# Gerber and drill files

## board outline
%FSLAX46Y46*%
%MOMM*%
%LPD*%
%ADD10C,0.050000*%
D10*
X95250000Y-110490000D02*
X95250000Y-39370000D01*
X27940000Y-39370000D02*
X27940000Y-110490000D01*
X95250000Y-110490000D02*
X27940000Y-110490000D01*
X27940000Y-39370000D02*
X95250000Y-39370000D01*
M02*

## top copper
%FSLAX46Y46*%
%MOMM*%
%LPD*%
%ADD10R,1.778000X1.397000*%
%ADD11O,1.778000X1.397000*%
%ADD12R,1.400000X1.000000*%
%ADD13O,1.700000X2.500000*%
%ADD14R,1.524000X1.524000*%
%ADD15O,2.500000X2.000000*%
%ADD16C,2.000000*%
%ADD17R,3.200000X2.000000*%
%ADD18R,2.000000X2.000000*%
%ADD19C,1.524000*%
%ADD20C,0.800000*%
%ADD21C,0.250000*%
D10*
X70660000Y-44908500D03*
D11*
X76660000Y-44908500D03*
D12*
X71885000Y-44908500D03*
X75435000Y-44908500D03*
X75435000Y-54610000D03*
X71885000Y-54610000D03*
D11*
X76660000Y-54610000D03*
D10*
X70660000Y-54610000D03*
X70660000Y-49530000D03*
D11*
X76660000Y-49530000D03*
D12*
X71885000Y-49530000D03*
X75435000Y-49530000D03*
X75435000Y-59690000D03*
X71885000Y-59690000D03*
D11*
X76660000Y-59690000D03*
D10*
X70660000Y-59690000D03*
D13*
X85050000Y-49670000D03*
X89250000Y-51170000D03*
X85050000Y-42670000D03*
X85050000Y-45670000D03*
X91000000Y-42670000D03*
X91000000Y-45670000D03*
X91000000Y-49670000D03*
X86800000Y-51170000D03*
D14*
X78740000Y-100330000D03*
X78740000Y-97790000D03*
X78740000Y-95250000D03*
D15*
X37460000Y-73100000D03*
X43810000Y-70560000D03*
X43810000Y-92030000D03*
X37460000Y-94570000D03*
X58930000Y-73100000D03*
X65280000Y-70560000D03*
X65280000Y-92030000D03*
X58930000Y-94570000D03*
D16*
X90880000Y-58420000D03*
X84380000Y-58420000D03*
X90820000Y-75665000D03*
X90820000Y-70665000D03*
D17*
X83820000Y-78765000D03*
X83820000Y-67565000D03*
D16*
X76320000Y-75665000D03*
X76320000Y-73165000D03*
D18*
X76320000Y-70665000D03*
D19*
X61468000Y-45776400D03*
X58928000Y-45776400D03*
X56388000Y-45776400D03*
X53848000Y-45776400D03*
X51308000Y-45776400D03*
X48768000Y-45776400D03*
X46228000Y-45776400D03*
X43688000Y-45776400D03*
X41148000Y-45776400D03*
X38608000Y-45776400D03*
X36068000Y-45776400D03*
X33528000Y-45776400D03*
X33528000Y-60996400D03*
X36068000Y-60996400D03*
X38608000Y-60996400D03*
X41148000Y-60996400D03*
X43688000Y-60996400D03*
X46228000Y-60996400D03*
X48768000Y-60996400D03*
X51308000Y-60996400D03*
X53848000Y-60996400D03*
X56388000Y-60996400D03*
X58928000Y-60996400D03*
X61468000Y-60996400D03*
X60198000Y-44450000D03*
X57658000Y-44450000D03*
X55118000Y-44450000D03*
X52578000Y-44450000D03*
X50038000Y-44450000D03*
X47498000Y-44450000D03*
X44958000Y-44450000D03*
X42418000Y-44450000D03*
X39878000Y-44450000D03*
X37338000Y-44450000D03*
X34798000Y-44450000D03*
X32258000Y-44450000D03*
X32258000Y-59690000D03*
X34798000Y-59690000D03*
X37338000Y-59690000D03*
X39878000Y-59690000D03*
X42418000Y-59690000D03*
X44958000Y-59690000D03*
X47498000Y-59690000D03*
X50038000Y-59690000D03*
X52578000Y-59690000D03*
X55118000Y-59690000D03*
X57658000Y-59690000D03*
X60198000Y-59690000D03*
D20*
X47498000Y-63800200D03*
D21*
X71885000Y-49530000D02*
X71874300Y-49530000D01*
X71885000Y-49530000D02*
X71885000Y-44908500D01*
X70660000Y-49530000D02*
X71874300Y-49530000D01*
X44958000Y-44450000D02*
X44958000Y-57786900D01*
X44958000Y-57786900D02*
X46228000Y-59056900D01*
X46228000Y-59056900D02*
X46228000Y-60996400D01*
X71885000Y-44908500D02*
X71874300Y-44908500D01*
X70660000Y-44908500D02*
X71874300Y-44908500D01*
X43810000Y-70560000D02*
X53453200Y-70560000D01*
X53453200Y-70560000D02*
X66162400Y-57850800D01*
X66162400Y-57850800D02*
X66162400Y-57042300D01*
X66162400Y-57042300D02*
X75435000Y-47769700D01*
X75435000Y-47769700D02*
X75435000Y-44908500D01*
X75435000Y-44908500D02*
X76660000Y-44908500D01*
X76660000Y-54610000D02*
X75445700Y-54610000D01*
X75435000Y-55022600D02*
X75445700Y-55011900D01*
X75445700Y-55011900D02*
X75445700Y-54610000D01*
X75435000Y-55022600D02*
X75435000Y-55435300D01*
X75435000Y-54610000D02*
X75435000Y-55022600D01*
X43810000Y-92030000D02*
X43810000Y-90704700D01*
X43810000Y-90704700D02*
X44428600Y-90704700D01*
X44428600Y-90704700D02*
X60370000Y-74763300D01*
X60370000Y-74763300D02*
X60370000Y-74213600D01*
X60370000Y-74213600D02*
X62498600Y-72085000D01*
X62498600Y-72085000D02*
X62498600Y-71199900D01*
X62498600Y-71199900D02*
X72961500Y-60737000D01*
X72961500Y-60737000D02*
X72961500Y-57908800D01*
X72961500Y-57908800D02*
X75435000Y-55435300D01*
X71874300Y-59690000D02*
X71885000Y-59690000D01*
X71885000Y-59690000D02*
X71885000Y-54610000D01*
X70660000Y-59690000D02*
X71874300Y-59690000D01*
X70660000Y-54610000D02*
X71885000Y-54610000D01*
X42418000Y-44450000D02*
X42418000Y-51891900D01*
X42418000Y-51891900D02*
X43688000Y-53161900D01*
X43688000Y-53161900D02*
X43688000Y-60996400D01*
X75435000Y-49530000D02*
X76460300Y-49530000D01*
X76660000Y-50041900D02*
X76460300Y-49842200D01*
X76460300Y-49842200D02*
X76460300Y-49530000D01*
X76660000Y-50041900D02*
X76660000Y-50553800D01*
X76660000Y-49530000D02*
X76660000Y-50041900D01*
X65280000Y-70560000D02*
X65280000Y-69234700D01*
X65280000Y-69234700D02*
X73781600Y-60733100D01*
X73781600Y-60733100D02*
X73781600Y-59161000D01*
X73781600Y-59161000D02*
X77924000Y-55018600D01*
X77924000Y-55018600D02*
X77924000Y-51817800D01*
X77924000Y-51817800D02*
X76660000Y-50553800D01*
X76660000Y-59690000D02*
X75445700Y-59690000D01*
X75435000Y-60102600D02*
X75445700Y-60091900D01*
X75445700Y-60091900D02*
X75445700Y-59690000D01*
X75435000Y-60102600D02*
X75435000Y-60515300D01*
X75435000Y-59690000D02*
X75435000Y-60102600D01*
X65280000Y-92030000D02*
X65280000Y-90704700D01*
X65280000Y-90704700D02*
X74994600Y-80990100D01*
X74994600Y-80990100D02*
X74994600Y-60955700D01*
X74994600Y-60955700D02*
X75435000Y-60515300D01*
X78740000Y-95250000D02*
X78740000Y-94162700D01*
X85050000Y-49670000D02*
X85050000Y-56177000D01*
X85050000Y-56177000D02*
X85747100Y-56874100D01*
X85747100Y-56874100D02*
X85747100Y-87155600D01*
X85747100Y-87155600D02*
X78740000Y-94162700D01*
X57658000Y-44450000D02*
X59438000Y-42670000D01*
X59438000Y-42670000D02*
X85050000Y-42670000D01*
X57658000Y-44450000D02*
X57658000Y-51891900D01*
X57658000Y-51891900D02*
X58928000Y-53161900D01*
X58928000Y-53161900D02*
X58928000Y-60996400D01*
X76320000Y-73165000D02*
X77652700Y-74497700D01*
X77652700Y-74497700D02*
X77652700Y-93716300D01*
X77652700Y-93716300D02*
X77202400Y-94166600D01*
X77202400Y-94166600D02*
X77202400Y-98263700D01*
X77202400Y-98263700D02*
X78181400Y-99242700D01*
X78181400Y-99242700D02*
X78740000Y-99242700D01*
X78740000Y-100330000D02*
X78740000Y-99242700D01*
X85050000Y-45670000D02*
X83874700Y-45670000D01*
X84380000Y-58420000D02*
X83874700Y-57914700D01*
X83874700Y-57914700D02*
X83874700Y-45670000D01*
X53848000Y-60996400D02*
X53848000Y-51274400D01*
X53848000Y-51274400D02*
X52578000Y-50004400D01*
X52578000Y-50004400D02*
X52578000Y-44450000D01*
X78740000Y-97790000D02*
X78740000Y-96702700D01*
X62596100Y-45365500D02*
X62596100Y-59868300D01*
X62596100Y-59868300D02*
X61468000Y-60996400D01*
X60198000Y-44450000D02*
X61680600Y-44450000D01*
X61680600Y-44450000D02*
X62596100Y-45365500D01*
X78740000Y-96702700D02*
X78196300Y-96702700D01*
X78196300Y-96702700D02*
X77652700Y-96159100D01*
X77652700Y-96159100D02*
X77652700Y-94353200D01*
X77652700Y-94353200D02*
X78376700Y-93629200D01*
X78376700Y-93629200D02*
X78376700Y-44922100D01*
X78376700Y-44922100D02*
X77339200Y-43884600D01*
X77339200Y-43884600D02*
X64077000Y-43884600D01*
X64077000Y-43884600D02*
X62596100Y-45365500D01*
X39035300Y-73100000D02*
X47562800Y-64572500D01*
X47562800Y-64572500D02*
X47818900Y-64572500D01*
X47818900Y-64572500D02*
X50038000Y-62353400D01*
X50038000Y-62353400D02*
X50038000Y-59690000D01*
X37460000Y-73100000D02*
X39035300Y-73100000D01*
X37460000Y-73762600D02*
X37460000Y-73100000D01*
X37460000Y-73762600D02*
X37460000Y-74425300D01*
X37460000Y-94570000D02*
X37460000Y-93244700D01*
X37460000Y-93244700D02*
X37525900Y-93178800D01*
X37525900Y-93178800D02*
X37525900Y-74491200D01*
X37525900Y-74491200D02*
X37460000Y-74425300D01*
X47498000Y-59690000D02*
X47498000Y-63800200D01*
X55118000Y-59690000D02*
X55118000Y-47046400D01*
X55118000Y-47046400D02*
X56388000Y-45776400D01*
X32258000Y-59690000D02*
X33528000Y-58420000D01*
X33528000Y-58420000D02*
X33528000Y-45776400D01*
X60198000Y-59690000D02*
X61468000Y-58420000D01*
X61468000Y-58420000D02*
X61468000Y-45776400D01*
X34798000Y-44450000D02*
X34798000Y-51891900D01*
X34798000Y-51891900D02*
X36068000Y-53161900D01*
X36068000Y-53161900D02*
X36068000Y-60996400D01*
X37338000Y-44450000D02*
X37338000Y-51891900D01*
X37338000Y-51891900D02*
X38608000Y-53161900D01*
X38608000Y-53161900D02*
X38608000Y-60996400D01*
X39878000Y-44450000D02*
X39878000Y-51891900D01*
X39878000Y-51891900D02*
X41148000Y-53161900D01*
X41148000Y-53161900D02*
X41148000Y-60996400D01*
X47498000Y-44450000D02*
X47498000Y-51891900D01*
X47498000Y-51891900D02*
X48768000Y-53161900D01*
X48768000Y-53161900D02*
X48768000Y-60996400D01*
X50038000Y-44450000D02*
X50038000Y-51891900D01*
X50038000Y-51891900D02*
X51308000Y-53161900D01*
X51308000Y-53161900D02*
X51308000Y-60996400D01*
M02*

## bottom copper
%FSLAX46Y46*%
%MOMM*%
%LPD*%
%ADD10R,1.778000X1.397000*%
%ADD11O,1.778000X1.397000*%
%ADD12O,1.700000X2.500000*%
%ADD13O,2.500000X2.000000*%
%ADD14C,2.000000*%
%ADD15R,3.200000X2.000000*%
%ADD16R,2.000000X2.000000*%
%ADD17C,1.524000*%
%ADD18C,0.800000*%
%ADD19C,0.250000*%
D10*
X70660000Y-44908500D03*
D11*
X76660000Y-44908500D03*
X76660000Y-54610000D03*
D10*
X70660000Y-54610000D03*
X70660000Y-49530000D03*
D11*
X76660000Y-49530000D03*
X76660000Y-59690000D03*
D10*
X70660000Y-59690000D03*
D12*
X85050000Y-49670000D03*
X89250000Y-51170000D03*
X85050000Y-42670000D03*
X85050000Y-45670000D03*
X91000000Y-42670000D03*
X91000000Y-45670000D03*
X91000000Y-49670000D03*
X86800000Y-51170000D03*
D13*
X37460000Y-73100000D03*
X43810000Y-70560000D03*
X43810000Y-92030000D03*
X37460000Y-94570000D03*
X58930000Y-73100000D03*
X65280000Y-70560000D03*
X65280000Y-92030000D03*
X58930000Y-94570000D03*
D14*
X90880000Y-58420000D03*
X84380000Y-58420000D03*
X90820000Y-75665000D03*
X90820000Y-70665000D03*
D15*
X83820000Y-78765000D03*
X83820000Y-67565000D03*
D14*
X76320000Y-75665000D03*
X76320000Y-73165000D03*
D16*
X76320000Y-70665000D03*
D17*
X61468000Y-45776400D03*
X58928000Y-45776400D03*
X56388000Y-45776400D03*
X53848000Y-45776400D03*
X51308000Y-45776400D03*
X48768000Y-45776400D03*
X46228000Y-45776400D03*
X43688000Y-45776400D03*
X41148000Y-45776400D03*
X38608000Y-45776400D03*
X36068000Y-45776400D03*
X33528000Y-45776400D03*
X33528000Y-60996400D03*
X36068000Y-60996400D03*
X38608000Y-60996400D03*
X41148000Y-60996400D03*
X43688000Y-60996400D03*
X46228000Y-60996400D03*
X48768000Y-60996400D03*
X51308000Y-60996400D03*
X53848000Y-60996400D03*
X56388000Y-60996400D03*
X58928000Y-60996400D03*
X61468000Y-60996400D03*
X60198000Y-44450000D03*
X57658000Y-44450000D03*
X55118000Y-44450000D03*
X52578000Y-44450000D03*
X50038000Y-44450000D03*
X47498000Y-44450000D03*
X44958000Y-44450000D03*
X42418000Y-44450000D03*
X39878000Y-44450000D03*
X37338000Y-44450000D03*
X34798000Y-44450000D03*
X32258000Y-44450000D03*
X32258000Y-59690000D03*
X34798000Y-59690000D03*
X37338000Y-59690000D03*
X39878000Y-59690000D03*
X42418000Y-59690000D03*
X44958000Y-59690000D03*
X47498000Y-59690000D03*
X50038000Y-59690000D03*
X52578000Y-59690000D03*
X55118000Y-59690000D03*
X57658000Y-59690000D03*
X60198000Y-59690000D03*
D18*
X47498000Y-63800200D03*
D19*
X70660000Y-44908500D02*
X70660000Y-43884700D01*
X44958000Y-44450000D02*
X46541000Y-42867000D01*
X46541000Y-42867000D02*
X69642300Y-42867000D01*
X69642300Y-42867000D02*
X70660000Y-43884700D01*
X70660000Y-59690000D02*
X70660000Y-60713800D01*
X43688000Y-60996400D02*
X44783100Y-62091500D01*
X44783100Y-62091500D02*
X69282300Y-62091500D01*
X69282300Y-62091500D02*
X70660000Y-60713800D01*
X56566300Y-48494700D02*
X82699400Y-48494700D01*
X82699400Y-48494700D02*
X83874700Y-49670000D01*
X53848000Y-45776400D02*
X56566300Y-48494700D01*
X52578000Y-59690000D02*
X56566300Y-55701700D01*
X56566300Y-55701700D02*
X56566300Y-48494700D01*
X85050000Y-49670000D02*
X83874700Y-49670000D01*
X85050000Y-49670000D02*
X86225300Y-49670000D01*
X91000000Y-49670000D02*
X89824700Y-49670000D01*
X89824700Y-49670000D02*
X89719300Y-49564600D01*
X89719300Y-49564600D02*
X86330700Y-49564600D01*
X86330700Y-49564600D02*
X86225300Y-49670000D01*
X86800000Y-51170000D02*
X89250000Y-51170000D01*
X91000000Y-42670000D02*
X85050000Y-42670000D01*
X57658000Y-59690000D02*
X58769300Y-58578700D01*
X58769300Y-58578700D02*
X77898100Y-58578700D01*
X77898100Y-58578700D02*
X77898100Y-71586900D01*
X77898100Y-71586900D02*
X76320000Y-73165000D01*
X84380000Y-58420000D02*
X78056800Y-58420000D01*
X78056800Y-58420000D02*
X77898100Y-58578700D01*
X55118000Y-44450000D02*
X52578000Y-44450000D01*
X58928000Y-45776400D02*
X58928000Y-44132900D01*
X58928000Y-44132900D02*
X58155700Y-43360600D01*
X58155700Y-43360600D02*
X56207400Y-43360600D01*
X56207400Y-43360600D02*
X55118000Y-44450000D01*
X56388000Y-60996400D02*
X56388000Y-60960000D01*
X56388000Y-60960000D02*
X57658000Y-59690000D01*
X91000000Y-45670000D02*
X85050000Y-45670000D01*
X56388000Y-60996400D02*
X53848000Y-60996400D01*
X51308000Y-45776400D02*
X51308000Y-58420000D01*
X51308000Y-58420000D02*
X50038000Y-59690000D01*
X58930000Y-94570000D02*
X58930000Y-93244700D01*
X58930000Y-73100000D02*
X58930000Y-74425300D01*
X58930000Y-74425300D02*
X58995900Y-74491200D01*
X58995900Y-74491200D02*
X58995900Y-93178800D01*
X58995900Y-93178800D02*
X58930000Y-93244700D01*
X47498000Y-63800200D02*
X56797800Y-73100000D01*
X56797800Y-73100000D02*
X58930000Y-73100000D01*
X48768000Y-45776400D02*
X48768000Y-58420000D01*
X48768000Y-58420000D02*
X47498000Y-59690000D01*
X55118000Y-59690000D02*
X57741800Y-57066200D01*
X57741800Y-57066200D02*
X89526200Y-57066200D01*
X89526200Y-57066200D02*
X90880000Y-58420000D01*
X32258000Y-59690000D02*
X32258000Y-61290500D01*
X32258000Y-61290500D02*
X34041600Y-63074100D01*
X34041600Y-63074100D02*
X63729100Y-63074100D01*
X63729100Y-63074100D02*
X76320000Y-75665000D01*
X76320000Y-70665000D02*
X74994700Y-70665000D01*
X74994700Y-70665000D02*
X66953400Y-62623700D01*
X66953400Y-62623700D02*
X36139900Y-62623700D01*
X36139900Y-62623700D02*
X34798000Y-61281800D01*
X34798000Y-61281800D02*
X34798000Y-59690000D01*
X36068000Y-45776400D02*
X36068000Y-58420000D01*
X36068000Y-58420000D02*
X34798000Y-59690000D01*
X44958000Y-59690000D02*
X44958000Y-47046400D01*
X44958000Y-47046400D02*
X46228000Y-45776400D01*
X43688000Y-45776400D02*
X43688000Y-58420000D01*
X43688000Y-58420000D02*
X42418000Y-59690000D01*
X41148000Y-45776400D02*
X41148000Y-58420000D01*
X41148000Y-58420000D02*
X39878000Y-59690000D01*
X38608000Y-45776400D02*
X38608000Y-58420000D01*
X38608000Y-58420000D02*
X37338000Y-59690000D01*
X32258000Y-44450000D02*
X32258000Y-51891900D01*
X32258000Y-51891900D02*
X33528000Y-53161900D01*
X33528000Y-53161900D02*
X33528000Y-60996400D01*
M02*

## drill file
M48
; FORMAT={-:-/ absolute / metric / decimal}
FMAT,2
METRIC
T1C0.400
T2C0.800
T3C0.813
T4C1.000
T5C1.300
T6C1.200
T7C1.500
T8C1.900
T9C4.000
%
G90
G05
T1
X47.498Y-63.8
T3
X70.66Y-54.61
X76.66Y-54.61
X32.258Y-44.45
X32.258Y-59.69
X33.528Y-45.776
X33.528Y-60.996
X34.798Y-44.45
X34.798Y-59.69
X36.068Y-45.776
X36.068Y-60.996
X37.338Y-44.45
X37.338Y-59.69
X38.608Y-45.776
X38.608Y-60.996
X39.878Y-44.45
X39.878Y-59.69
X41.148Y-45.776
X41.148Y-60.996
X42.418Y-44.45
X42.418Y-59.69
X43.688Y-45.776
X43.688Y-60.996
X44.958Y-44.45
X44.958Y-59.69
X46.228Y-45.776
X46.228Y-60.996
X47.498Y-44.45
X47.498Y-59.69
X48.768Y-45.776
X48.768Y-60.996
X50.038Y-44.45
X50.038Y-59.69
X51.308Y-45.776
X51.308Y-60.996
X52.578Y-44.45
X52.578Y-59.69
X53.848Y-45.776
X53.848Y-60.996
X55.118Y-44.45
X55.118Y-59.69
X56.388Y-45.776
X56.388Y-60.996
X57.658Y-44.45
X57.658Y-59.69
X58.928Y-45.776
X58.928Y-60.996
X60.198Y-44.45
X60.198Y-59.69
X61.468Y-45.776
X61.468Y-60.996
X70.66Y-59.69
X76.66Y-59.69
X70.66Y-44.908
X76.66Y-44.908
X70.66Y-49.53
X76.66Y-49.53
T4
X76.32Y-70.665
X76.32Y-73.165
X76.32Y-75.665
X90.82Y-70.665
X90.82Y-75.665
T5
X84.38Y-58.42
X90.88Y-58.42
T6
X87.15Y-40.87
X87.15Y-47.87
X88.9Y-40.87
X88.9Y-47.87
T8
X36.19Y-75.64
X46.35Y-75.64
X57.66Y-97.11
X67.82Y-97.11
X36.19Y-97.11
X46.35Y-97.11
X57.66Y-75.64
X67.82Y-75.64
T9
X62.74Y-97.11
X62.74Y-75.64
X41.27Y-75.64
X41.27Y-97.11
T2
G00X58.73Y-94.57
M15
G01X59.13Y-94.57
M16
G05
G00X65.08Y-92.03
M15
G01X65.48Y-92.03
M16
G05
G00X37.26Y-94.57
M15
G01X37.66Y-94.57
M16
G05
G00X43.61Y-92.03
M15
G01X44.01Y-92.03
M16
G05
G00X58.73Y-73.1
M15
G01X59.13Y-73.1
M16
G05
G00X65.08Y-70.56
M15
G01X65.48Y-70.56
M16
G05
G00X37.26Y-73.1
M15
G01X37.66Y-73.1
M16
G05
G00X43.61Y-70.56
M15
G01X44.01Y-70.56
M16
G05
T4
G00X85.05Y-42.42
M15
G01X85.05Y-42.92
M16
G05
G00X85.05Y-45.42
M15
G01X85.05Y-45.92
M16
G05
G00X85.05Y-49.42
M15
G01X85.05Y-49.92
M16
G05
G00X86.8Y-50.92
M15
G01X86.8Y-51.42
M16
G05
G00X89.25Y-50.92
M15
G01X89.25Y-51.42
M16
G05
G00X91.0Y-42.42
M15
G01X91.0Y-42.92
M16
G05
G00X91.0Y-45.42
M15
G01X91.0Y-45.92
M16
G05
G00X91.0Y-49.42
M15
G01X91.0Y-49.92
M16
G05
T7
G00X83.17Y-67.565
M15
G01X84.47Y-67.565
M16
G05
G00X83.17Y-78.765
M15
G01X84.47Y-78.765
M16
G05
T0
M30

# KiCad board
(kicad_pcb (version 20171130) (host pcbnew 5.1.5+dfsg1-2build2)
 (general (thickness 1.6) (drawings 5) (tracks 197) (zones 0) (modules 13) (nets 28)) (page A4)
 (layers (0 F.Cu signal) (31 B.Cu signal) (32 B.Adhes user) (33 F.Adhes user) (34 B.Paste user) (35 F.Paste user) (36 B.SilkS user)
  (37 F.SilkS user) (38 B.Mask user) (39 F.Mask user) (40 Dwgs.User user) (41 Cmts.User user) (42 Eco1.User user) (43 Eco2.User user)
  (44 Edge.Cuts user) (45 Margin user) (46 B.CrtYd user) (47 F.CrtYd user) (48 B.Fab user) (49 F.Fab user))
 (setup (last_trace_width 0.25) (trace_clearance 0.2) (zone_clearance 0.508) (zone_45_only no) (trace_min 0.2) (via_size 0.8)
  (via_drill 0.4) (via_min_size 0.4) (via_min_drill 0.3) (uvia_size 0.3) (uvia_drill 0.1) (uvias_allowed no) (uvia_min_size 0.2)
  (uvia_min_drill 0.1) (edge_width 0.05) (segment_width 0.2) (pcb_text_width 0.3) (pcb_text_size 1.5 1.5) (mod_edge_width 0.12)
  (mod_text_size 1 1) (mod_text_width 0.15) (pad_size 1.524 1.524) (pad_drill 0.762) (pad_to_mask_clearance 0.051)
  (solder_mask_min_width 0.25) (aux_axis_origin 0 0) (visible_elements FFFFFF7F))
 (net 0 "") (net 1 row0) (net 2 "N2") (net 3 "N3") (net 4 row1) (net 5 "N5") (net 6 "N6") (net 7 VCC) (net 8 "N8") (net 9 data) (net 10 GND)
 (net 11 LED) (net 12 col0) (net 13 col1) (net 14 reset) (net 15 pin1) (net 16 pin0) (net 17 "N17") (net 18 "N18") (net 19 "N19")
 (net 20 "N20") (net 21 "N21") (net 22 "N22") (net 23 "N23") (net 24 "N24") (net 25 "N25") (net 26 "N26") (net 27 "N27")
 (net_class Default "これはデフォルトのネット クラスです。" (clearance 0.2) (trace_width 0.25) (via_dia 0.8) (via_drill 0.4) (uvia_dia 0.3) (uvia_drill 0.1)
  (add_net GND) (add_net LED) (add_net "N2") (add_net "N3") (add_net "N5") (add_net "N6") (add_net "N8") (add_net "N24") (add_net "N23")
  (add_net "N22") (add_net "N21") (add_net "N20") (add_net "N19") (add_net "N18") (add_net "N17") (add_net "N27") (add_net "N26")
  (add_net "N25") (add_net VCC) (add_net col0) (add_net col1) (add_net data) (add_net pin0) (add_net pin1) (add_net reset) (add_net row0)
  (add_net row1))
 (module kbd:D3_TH (layer F.Cu) (at 73.66 44.9085) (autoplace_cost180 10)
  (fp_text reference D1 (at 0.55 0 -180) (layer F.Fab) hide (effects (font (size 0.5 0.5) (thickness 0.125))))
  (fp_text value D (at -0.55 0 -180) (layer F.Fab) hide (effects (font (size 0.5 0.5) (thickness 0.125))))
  (pad 1 thru_hole rect (at -3 0) (size 1.778 1.397) (drill 0.8128) (layers *.Cu B.Mask) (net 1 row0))
  (pad 2 thru_hole oval (at 3 0) (size 1.778 1.397) (drill 0.8128) (layers *.Cu B.Mask) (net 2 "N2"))
  (pad 1 smd rect (at -1.775 0 180) (size 1.4 1) (layers F.Cu F.Paste F.Mask) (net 1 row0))
  (pad 2 smd rect (at 1.775 0 180) (size 1.4 1) (layers F.Cu F.Paste F.Mask) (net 2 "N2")))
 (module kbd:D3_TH (layer F.Cu) (at 73.66 54.61) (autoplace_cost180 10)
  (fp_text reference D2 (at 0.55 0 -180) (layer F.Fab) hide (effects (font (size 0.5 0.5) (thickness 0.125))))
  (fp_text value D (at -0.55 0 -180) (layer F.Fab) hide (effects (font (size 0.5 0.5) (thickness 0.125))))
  (pad 2 smd rect (at 1.775 0 180) (size 1.4 1) (layers F.Cu F.Paste F.Mask) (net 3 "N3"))
  (pad 1 smd rect (at -1.775 0 180) (size 1.4 1) (layers F.Cu F.Paste F.Mask) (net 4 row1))
  (pad 2 thru_hole oval (at 3 0) (size 1.778 1.397) (drill 0.8128) (layers *.Cu B.Mask) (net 3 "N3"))
  (pad 1 thru_hole rect (at -3 0) (size 1.778 1.397) (drill 0.8128) (layers *.Cu B.Mask) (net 4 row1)))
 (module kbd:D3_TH (layer F.Cu) (at 73.66 49.53) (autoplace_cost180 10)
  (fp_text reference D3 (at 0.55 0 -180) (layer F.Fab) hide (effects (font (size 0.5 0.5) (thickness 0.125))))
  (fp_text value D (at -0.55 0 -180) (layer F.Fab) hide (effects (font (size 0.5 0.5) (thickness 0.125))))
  (pad 1 thru_hole rect (at -3 0) (size 1.778 1.397) (drill 0.8128) (layers *.Cu B.Mask) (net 1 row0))
  (pad 2 thru_hole oval (at 3 0) (size 1.778 1.397) (drill 0.8128) (layers *.Cu B.Mask) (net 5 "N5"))
  (pad 1 smd rect (at -1.775 0 180) (size 1.4 1) (layers F.Cu F.Paste F.Mask) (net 1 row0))
  (pad 2 smd rect (at 1.775 0 180) (size 1.4 1) (layers F.Cu F.Paste F.Mask) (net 5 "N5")))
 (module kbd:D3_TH (layer F.Cu) (at 73.66 59.69) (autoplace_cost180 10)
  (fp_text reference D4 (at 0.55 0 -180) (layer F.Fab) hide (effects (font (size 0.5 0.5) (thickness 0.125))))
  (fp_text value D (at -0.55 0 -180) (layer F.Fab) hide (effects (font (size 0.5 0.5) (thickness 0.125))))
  (pad 2 smd rect (at 1.775 0 180) (size 1.4 1) (layers F.Cu F.Paste F.Mask) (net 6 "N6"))
  (pad 1 smd rect (at -1.775 0 180) (size 1.4 1) (layers F.Cu F.Paste F.Mask) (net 4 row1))
  (pad 2 thru_hole oval (at 3 0) (size 1.778 1.397) (drill 0.8128) (layers *.Cu B.Mask) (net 6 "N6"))
  (pad 1 thru_hole rect (at -3 0) (size 1.778 1.397) (drill 0.8128) (layers *.Cu B.Mask) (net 4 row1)))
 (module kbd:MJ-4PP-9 (layer F.Cu) (at 88.9 39.37)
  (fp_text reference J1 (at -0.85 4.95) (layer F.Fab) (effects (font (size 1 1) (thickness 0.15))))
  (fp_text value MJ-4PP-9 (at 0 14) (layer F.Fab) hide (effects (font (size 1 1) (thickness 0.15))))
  (pad "" np_thru_hole circle (at -1.75 8.5) (size 1.2 1.2) (drill 1.2) (layers *.Cu *.Mask F.SilkS))
  (pad "" np_thru_hole circle (at -1.75 1.5) (size 1.2 1.2) (drill 1.2) (layers *.Cu *.Mask F.SilkS))
  (pad D thru_hole oval (at -3.85 10.3) (size 1.7 2.5) (drill oval 1 1.5) (layers *.Cu *.Mask F.SilkS) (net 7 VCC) (clearance 0.15))
  (pad A thru_hole oval (at 0.35 11.8) (size 1.7 2.5) (drill oval 1 1.5) (layers *.Cu *.Mask F.SilkS) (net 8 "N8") (clearance 0.15))
  (pad B thru_hole oval (at -3.85 3.3) (size 1.7 2.5) (drill oval 1 1.5) (layers *.Cu *.Mask F.SilkS) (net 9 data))
  (pad C thru_hole oval (at -3.85 6.3) (size 1.7 2.5) (drill oval 1 1.5) (layers *.Cu *.Mask F.SilkS) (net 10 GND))
  (pad "" np_thru_hole circle (at 0 1.5) (size 1.2 1.2) (drill 1.2) (layers *.Cu *.Mask F.SilkS))
  (pad "" np_thru_hole circle (at 0 8.5) (size 1.2 1.2) (drill 1.2) (layers *.Cu *.Mask F.SilkS))
  (pad B thru_hole oval (at 2.1 3.3) (size 1.7 2.5) (drill oval 1 1.5) (layers *.Cu *.Mask F.SilkS) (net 9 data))
  (pad C thru_hole oval (at 2.1 6.3) (size 1.7 2.5) (drill oval 1 1.5) (layers *.Cu *.Mask F.SilkS) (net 10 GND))
  (pad D thru_hole oval (at 2.1 10.3) (size 1.7 2.5) (drill oval 1 1.5) (layers *.Cu *.Mask F.SilkS) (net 7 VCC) (clearance 0.15))
  (pad A thru_hole oval (at -2.1 11.8) (size 1.7 2.5) (drill oval 1 1.5) (layers *.Cu *.Mask F.SilkS) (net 8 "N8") (clearance 0.15)))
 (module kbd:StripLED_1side (layer F.Cu) (at 78.74 95.25)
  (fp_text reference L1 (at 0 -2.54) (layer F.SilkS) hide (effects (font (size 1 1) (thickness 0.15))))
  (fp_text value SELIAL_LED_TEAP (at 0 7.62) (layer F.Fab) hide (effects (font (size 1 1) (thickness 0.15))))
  (pad 3 smd rect (at 0 5.08) (size 1.524 1.524) (layers F.Cu F.Mask) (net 10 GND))
  (pad 2 smd rect (at 0 2.54) (size 1.524 1.524) (layers F.Cu F.Mask) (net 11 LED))
  (pad 1 smd rect (at 0 0) (size 1.524 1.524) (layers F.Cu F.Mask) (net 7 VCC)))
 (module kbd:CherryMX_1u (layer F.Cu) (at 41.27 75.64)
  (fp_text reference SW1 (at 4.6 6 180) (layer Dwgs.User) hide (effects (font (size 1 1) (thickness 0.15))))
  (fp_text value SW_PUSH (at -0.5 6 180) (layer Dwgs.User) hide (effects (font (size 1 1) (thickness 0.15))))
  (pad 1 thru_hole oval (at -3.81 -2.54) (size 2.5 2) (drill oval 1.2 0.8) (layers *.Cu F.SilkS B.Mask) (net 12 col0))
  (pad 2 thru_hole oval (at 2.54 -5.08) (size 2.5 2) (drill oval 1.2 0.8) (layers *.Cu F.SilkS B.Mask) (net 2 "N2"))
  (pad "" np_thru_hole circle (at 5.08 0 90) (size 1.9 1.9) (drill 1.9) (layers *.Cu *.Mask))
  (pad "" np_thru_hole circle (at -5.08 0 90) (size 1.9 1.9) (drill 1.9) (layers *.Cu *.Mask))
  (pad "" np_thru_hole circle (at 0 0 90) (size 4 4) (drill 4) (layers *.Cu *.Mask)))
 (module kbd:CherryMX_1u (layer F.Cu) (at 41.27 97.11)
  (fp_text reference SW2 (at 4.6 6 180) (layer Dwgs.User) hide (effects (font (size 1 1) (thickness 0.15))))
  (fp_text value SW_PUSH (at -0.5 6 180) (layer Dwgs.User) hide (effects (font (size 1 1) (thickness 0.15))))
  (pad "" np_thru_hole circle (at 0 0 90) (size 4 4) (drill 4) (layers *.Cu *.Mask))
  (pad "" np_thru_hole circle (at -5.08 0 90) (size 1.9 1.9) (drill 1.9) (layers *.Cu *.Mask))
  (pad "" np_thru_hole circle (at 5.08 0 90) (size 1.9 1.9) (drill 1.9) (layers *.Cu *.Mask))
  (pad 2 thru_hole oval (at 2.54 -5.08) (size 2.5 2) (drill oval 1.2 0.8) (layers *.Cu F.SilkS B.Mask) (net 3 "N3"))
  (pad 1 thru_hole oval (at -3.81 -2.54) (size 2.5 2) (drill oval 1.2 0.8) (layers *.Cu F.SilkS B.Mask) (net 12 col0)))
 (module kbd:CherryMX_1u (layer F.Cu) (at 62.74 75.64)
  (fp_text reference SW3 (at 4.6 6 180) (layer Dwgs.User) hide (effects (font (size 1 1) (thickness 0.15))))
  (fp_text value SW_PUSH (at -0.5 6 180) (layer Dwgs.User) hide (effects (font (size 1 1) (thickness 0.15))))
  (pad 1 thru_hole oval (at -3.81 -2.54) (size 2.5 2) (drill oval 1.2 0.8) (layers *.Cu F.SilkS B.Mask) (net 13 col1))
  (pad 2 thru_hole oval (at 2.54 -5.08) (size 2.5 2) (drill oval 1.2 0.8) (layers *.Cu F.SilkS B.Mask) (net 5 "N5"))
  (pad "" np_thru_hole circle (at 5.08 0 90) (size 1.9 1.9) (drill 1.9) (layers *.Cu *.Mask))
  (pad "" np_thru_hole circle (at -5.08 0 90) (size 1.9 1.9) (drill 1.9) (layers *.Cu *.Mask))
  (pad "" np_thru_hole circle (at 0 0 90) (size 4 4) (drill 4) (layers *.Cu *.Mask)))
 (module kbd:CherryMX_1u (layer F.Cu) (at 62.74 97.11)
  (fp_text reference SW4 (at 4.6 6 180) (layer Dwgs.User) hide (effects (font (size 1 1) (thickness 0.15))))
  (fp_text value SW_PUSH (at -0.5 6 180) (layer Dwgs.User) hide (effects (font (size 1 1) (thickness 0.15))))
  (pad "" np_thru_hole circle (at 0 0 90) (size 4 4) (drill 4) (layers *.Cu *.Mask))
  (pad "" np_thru_hole circle (at -5.08 0 90) (size 1.9 1.9) (drill 1.9) (layers *.Cu *.Mask))
  (pad "" np_thru_hole circle (at 5.08 0 90) (size 1.9 1.9) (drill 1.9) (layers *.Cu *.Mask))
  (pad 2 thru_hole oval (at 2.54 -5.08) (size 2.5 2) (drill oval 1.2 0.8) (layers *.Cu F.SilkS B.Mask) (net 6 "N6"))
  (pad 1 thru_hole oval (at -3.81 -2.54) (size 2.5 2) (drill oval 1.2 0.8) (layers *.Cu F.SilkS B.Mask) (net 13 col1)))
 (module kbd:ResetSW (layer F.Cu) (at 87.63 58.42)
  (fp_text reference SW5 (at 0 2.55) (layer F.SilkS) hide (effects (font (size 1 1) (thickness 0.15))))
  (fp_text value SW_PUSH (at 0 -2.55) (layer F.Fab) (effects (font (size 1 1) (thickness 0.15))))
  (pad 1 thru_hole circle (at 3.25 0) (size 2 2) (drill 1.3) (layers *.Cu *.Mask F.SilkS) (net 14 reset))
  (pad 2 thru_hole circle (at -3.25 0) (size 2 2) (drill 1.3) (layers *.Cu *.Mask F.SilkS) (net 10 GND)))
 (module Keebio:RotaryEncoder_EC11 (layer F.Cu) (at 83.82 73.165)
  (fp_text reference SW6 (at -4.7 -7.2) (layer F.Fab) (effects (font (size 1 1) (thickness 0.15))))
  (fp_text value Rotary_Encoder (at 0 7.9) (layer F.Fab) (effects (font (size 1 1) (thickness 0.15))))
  (pad S1 thru_hole circle (at 7 2.5) (size 2 2) (drill 1) (layers *.Cu *.Mask))
  (pad S2 thru_hole circle (at 7 -2.5) (size 2 2) (drill 1) (layers *.Cu *.Mask))
  (pad "" np_thru_hole rect (at 0 5.6) (size 3.2 2) (drill oval 2.8 1.5) (layers *.Cu *.Mask))
  (pad "" np_thru_hole rect (at 0 -5.6) (size 3.2 2) (drill oval 2.8 1.5) (layers *.Cu *.Mask))
  (pad B thru_hole circle (at -7.5 2.5) (size 2 2) (drill 1) (layers *.Cu *.Mask) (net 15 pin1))
  (pad C thru_hole circle (at -7.5 0) (size 2 2) (drill 1) (layers *.Cu *.Mask) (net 10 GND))
  (pad A thru_hole rect (at -7.5 -2.5) (size 2 2) (drill 1) (layers *.Cu *.Mask) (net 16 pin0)))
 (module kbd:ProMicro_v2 (layer F.Cu) (at 46.99 53.34 270)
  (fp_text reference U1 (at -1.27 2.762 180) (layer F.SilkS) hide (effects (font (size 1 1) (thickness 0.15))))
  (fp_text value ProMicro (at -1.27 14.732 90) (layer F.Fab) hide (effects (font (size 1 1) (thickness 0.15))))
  (pad 24 thru_hole circle (at -7.5636 -14.478 270) (size 1.524 1.524) (drill 0.8128) (layers *.Cu *.Mask F.SilkS) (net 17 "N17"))
  (pad 23 thru_hole circle (at -7.5636 -11.938 270) (size 1.524 1.524) (drill 0.8128) (layers *.Cu *.Mask F.SilkS) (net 10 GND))
  (pad 22 thru_hole circle (at -7.5636 -9.398 270) (size 1.524 1.524) (drill 0.8128) (layers *.Cu *.Mask F.SilkS) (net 14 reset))
  (pad 21 thru_hole circle (at -7.5636 -6.858 270) (size 1.524 1.524) (drill 0.8128) (layers *.Cu *.Mask F.SilkS) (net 7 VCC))
  (pad 20 thru_hole circle (at -7.5636 -4.318 270) (size 1.524 1.524) (drill 0.8128) (layers *.Cu *.Mask F.SilkS) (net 12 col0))
  (pad 19 thru_hole circle (at -7.5636 -1.778 270) (size 1.524 1.524) (drill 0.8128) (layers *.Cu *.Mask F.SilkS) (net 13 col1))
  (pad 18 thru_hole circle (at -7.5636 0.762 270) (size 1.524 1.524) (drill 0.8128) (layers *.Cu *.Mask F.SilkS) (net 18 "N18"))
  (pad 17 thru_hole circle (at -7.5636 3.302 270) (size 1.524 1.524) (drill 0.8128) (layers *.Cu *.Mask F.SilkS) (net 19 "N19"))
  (pad 16 thru_hole circle (at -7.5636 5.842 270) (size 1.524 1.524) (drill 0.8128) (layers *.Cu *.Mask F.SilkS) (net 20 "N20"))
  (pad 15 thru_hole circle (at -7.5636 8.382 270) (size 1.524 1.524) (drill 0.8128) (layers *.Cu *.Mask F.SilkS) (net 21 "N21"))
  (pad 14 thru_hole circle (at -7.5636 10.922 270) (size 1.524 1.524) (drill 0.8128) (layers *.Cu *.Mask F.SilkS) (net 16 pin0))
  (pad 13 thru_hole circle (at -7.5636 13.462 270) (size 1.524 1.524) (drill 0.8128) (layers *.Cu *.Mask F.SilkS) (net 15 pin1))
  (pad 12 thru_hole circle (at 7.6564 13.462 270) (size 1.524 1.524) (drill 0.8128) (layers *.Cu *.Mask F.SilkS) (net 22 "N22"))
  (pad 11 thru_hole circle (at 7.6564 10.922 270) (size 1.524 1.524) (drill 0.8128) (layers *.Cu *.Mask F.SilkS) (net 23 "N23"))
  (pad 10 thru_hole circle (at 7.6564 8.382 270) (size 1.524 1.524) (drill 0.8128) (layers *.Cu *.Mask F.SilkS) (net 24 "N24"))
  (pad 9 thru_hole circle (at 7.6564 5.842 270) (size 1.524 1.524) (drill 0.8128) (layers *.Cu *.Mask F.SilkS) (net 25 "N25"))
  (pad 8 thru_hole circle (at 7.6564 3.302 270) (size 1.524 1.524) (drill 0.8128) (layers *.Cu *.Mask F.SilkS) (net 4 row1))
  (pad 7 thru_hole circle (at 7.6564 0.762 270) (size 1.524 1.524) (drill 0.8128) (layers *.Cu *.Mask F.SilkS) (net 1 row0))
  (pad 6 thru_hole circle (at 7.6564 -1.778 270) (size 1.524 1.524) (drill 0.8128) (layers *.Cu *.Mask F.SilkS) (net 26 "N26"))
  (pad 5 thru_hole circle (at 7.6564 -4.318 270) (size 1.524 1.524) (drill 0.8128) (layers *.Cu *.Mask F.SilkS) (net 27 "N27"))
  (pad 4 thru_hole circle (at 7.6564 -6.858 270) (size 1.524 1.524) (drill 0.8128) (layers *.Cu *.Mask F.SilkS) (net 10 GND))
  (pad 3 thru_hole circle (at 7.6564 -9.398 270) (size 1.524 1.524) (drill 0.8128) (layers *.Cu *.Mask F.SilkS) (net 10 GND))
  (pad 2 thru_hole circle (at 7.6564 -11.938 270) (size 1.524 1.524) (drill 0.8128) (layers *.Cu *.Mask F.SilkS) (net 9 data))
  (pad 1 thru_hole circle (at 7.6564 -14.478 270) (size 1.524 1.524) (drill 0.8128) (layers *.Cu *.Mask F.SilkS) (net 11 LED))
  (pad 1 thru_hole circle (at -8.89 -13.208 270) (size 1.524 1.524) (drill 0.8128) (layers *.Cu *.Mask F.SilkS) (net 11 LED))
  (pad 2 thru_hole circle (at -8.89 -10.668 270) (size 1.524 1.524) (drill 0.8128) (layers *.Cu *.Mask F.SilkS) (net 9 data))
  (pad 3 thru_hole circle (at -8.89 -8.128 270) (size 1.524 1.524) (drill 0.8128) (layers *.Cu *.Mask F.SilkS) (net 10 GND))
  (pad 4 thru_hole circle (at -8.89 -5.588 270) (size 1.524 1.524) (drill 0.8128) (layers *.Cu *.Mask F.SilkS) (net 10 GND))
  (pad 5 thru_hole circle (at -8.89 -3.048 270) (size 1.524 1.524) (drill 0.8128) (layers *.Cu *.Mask F.SilkS) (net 27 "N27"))
  (pad 6 thru_hole circle (at -8.89 -0.508 270) (size 1.524 1.524) (drill 0.8128) (layers *.Cu *.Mask F.SilkS) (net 26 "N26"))
  (pad 7 thru_hole circle (at -8.89 2.032 270) (size 1.524 1.524) (drill 0.8128) (layers *.Cu *.Mask F.SilkS) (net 1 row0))
  (pad 8 thru_hole circle (at -8.89 4.572 270) (size 1.524 1.524) (drill 0.8128) (layers *.Cu *.Mask F.SilkS) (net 4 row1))
  (pad 9 thru_hole circle (at -8.89 7.112 270) (size 1.524 1.524) (drill 0.8128) (layers *.Cu *.Mask F.SilkS) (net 25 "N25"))
  (pad 10 thru_hole circle (at -8.89 9.652 270) (size 1.524 1.524) (drill 0.8128) (layers *.Cu *.Mask F.SilkS) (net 24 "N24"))
  (pad 11 thru_hole circle (at -8.89 12.192 270) (size 1.524 1.524) (drill 0.8128) (layers *.Cu *.Mask F.SilkS) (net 23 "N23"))
  (pad 12 thru_hole circle (at -8.89 14.732 270) (size 1.524 1.524) (drill 0.8128) (layers *.Cu *.Mask F.SilkS) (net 22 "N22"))
  (pad 13 thru_hole circle (at 6.35 14.732 270) (size 1.524 1.524) (drill 0.8128) (layers *.Cu *.Mask F.SilkS) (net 15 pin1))
  (pad 14 thru_hole circle (at 6.35 12.192 270) (size 1.524 1.524) (drill 0.8128) (layers *.Cu *.Mask F.SilkS) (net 16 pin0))
  (pad 15 thru_hole circle (at 6.35 9.652 270) (size 1.524 1.524) (drill 0.8128) (layers *.Cu *.Mask F.SilkS) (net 21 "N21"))
  (pad 16 thru_hole circle (at 6.35 7.112 270) (size 1.524 1.524) (drill 0.8128) (layers *.Cu *.Mask F.SilkS) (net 20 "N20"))
  (pad 17 thru_hole circle (at 6.35 4.572 270) (size 1.524 1.524) (drill 0.8128) (layers *.Cu *.Mask F.SilkS) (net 19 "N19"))
  (pad 18 thru_hole circle (at 6.35 2.032 270) (size 1.524 1.524) (drill 0.8128) (layers *.Cu *.Mask F.SilkS) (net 18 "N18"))
  (pad 19 thru_hole circle (at 6.35 -0.508 270) (size 1.524 1.524) (drill 0.8128) (layers *.Cu *.Mask F.SilkS) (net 13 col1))
  (pad 20 thru_hole circle (at 6.35 -3.048 270) (size 1.524 1.524) (drill 0.8128) (layers *.Cu *.Mask F.SilkS) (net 12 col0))
  (pad 21 thru_hole circle (at 6.35 -5.588 270) (size 1.524 1.524) (drill 0.8128) (layers *.Cu *.Mask F.SilkS) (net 7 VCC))
  (pad 22 thru_hole circle (at 6.35 -8.128 270) (size 1.524 1.524) (drill 0.8128) (layers *.Cu *.Mask F.SilkS) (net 14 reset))
  (pad 23 thru_hole circle (at 6.35 -10.668 270) (size 1.524 1.524) (drill 0.8128) (layers *.Cu *.Mask F.SilkS) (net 10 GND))
  (pad 24 thru_hole circle (at 6.35 -13.208 270) (size 1.524 1.524) (drill 0.8128) (layers *.Cu *.Mask F.SilkS) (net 17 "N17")))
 (gr_line (start 95.25 110.49) (end 95.25 39.37) (layer Edge.Cuts) (width 0.05))
 (gr_line (start 27.94 39.37) (end 27.94 110.49) (layer Edge.Cuts) (width 0.05))
 (gr_line (start 95.25 110.49) (end 27.94 110.49) (layer Edge.Cuts) (width 0.05))
 (gr_line (start 27.94 39.37) (end 95.25 39.37) (layer Edge.Cuts) (width 0.05))
 (segment (start 71.885 49.53) (end 71.8743 49.53) (width 0.25) (layer F.Cu) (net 1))
 (segment (start 71.885 49.53) (end 71.885 44.9085) (width 0.25) (layer F.Cu) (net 1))
 (segment (start 70.66 49.53) (end 71.8743 49.53) (width 0.25) (layer F.Cu) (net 1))
 (segment (start 70.66 44.9085) (end 70.66 43.8847) (width 0.25) (layer B.Cu) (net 1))
 (segment (start 44.958 44.45) (end 46.541 42.867) (width 0.25) (layer B.Cu) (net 1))
 (segment (start 46.541 42.867) (end 69.6423 42.867) (width 0.25) (layer B.Cu) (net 1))
 (segment (start 69.6423 42.867) (end 70.66 43.8847) (width 0.25) (layer B.Cu) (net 1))
 (segment (start 44.958 44.45) (end 44.958 57.7869) (width 0.25) (layer F.Cu) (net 1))
 (segment (start 44.958 57.7869) (end 46.228 59.0569) (width 0.25) (layer F.Cu) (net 1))
 (segment (start 46.228 59.0569) (end 46.228 60.9964) (width 0.25) (layer F.Cu) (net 1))
 (segment (start 71.885 44.9085) (end 71.8743 44.9085) (width 0.25) (layer F.Cu) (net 1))
 (segment (start 70.66 44.9085) (end 71.8743 44.9085) (width 0.25) (layer F.Cu) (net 1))
 (segment (start 43.81 70.56) (end 53.4532 70.56) (width 0.25) (layer F.Cu) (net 2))
 (segment (start 53.4532 70.56) (end 66.1624 57.8508) (width 0.25) (layer F.Cu) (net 2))
 (segment (start 66.1624 57.8508) (end 66.1624 57.0423) (width 0.25) (layer F.Cu) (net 2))
 (segment (start 66.1624 57.0423) (end 75.435 47.7697) (width 0.25) (layer F.Cu) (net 2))
 (segment (start 75.435 47.7697) (end 75.435 44.9085) (width 0.25) (layer F.Cu) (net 2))
 (segment (start 75.435 44.9085) (end 76.66 44.9085) (width 0.25) (layer F.Cu) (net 2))
 (segment (start 76.66 54.61) (end 75.4457 54.61) (width 0.25) (layer F.Cu) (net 3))
 (segment (start 75.435 55.0226) (end 75.4457 55.0119) (width 0.25) (layer F.Cu) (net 3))
 (segment (start 75.4457 55.0119) (end 75.4457 54.61) (width 0.25) (layer F.Cu) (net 3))
 (segment (start 75.435 55.0226) (end 75.435 55.4353) (width 0.25) (layer F.Cu) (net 3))
 (segment (start 75.435 54.61) (end 75.435 55.0226) (width 0.25) (layer F.Cu) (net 3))
 (segment (start 43.81 92.03) (end 43.81 90.7047) (width 0.25) (layer F.Cu) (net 3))
 (segment (start 43.81 90.7047) (end 44.4286 90.7047) (width 0.25) (layer F.Cu) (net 3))
 (segment (start 44.4286 90.7047) (end 60.37 74.7633) (width 0.25) (layer F.Cu) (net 3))
 (segment (start 60.37 74.7633) (end 60.37 74.2136) (width 0.25) (layer F.Cu) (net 3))
 (segment (start 60.37 74.2136) (end 62.4986 72.085) (width 0.25) (layer F.Cu) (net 3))
 (segment (start 62.4986 72.085) (end 62.4986 71.1999) (width 0.25) (layer F.Cu) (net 3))
 (segment (start 62.4986 71.1999) (end 72.9615 60.737) (width 0.25) (layer F.Cu) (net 3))
 (segment (start 72.9615 60.737) (end 72.9615 57.9088) (width 0.25) (layer F.Cu) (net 3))
 (segment (start 72.9615 57.9088) (end 75.435 55.4353) (width 0.25) (layer F.Cu) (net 3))
 (segment (start 71.8743 59.69) (end 71.885 59.69) (width 0.25) (layer F.Cu) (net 4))
 (segment (start 71.885 59.69) (end 71.885 54.61) (width 0.25) (layer F.Cu) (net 4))
 (segment (start 70.66 59.69) (end 71.8743 59.69) (width 0.25) (layer F.Cu) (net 4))
 (segment (start 70.66 54.61) (end 71.885 54.61) (width 0.25) (layer F.Cu) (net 4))
 (segment (start 70.66 59.69) (end 70.66 60.7138) (width 0.25) (layer B.Cu) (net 4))
 (segment (start 43.688 60.9964) (end 44.7831 62.0915) (width 0.25) (layer B.Cu) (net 4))
 (segment (start 44.7831 62.0915) (end 69.2823 62.0915) (width 0.25) (layer B.Cu) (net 4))
 (segment (start 69.2823 62.0915) (end 70.66 60.7138) (width 0.25) (layer B.Cu) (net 4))
 (segment (start 42.418 44.45) (end 42.418 51.8919) (width 0.25) (layer F.Cu) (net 4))
 (segment (start 42.418 51.8919) (end 43.688 53.1619) (width 0.25) (layer F.Cu) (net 4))
 (segment (start 43.688 53.1619) (end 43.688 60.9964) (width 0.25) (layer F.Cu) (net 4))
 (segment (start 75.435 49.53) (end 76.4603 49.53) (width 0.25) (layer F.Cu) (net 5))
 (segment (start 76.66 50.0419) (end 76.4603 49.8422) (width 0.25) (layer F.Cu) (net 5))
 (segment (start 76.4603 49.8422) (end 76.4603 49.53) (width 0.25) (layer F.Cu) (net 5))
 (segment (start 76.66 50.0419) (end 76.66 50.5538) (width 0.25) (layer F.Cu) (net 5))
 (segment (start 76.66 49.53) (end 76.66 50.0419) (width 0.25) (layer F.Cu) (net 5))
 (segment (start 65.28 70.56) (end 65.28 69.2347) (width 0.25) (layer F.Cu) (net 5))
 (segment (start 65.28 69.2347) (end 73.7816 60.7331) (width 0.25) (layer F.Cu) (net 5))
 (segment (start 73.7816 60.7331) (end 73.7816 59.161) (width 0.25) (layer F.Cu) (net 5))
 (segment (start 73.7816 59.161) (end 77.924 55.0186) (width 0.25) (layer F.Cu) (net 5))
 (segment (start 77.924 55.0186) (end 77.924 51.8178) (width 0.25) (layer F.Cu) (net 5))
 (segment (start 77.924 51.8178) (end 76.66 50.5538) (width 0.25) (layer F.Cu) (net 5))
 (segment (start 76.66 59.69) (end 75.4457 59.69) (width 0.25) (layer F.Cu) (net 6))
 (segment (start 75.435 60.1026) (end 75.4457 60.0919) (width 0.25) (layer F.Cu) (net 6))
 (segment (start 75.4457 60.0919) (end 75.4457 59.69) (width 0.25) (layer F.Cu) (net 6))
 (segment (start 75.435 60.1026) (end 75.435 60.5153) (width 0.25) (layer F.Cu) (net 6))
 (segment (start 75.435 59.69) (end 75.435 60.1026) (width 0.25) (layer F.Cu) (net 6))
 (segment (start 65.28 92.03) (end 65.28 90.7047) (width 0.25) (layer F.Cu) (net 6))
 (segment (start 65.28 90.7047) (end 74.9946 80.9901) (width 0.25) (layer F.Cu) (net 6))
 (segment (start 74.9946 80.9901) (end 74.9946 60.9557) (width 0.25) (layer F.Cu) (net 6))
 (segment (start 74.9946 60.9557) (end 75.435 60.5153) (width 0.25) (layer F.Cu) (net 6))
 (segment (start 78.74 95.25) (end 78.74 94.1627) (width 0.25) (layer F.Cu) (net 7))
 (segment (start 85.05 49.67) (end 85.05 56.177) (width 0.25) (layer F.Cu) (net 7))
 (segment (start 85.05 56.177) (end 85.7471 56.8741) (width 0.25) (layer F.Cu) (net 7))
 (segment (start 85.7471 56.8741) (end 85.7471 87.1556) (width 0.25) (layer F.Cu) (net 7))
 (segment (start 85.7471 87.1556) (end 78.74 94.1627) (width 0.25) (layer F.Cu) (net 7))
 (segment (start 56.5663 48.4947) (end 82.6994 48.4947) (width 0.25) (layer B.Cu) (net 7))
 (segment (start 82.6994 48.4947) (end 83.8747 49.67) (width 0.25) (layer B.Cu) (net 7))
 (segment (start 53.848 45.7764) (end 56.5663 48.4947) (width 0.25) (layer B.Cu) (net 7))
 (segment (start 52.578 59.69) (end 56.5663 55.7017) (width 0.25) (layer B.Cu) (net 7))
 (segment (start 56.5663 55.7017) (end 56.5663 48.4947) (width 0.25) (layer B.Cu) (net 7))
 (segment (start 85.05 49.67) (end 83.8747 49.67) (width 0.25) (layer B.Cu) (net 7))
 (segment (start 85.05 49.67) (end 86.2253 49.67) (width 0.25) (layer B.Cu) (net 7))
 (segment (start 91 49.67) (end 89.8247 49.67) (width 0.25) (layer B.Cu) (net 7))
 (segment (start 89.8247 49.67) (end 89.7193 49.5646) (width 0.25) (layer B.Cu) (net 7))
 (segment (start 89.7193 49.5646) (end 86.3307 49.5646) (width 0.25) (layer B.Cu) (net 7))
 (segment (start 86.3307 49.5646) (end 86.2253 49.67) (width 0.25) (layer B.Cu) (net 7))
 (segment (start 86.8 51.17) (end 89.25 51.17) (width 0.25) (layer B.Cu) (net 8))
 (segment (start 57.658 44.45) (end 59.438 42.67) (width 0.25) (layer F.Cu) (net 9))
 (segment (start 59.438 42.67) (end 85.05 42.67) (width 0.25) (layer F.Cu) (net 9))
 (segment (start 57.658 44.45) (end 57.658 51.8919) (width 0.25) (layer F.Cu) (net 9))
 (segment (start 57.658 51.8919) (end 58.928 53.1619) (width 0.25) (layer F.Cu) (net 9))
 (segment (start 58.928 53.1619) (end 58.928 60.9964) (width 0.25) (layer F.Cu) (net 9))
 (segment (start 91 42.67) (end 85.05 42.67) (width 0.25) (layer B.Cu) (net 9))
 (segment (start 76.32 73.165) (end 77.6527 74.4977) (width 0.25) (layer F.Cu) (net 10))
 (segment (start 77.6527 74.4977) (end 77.6527 93.7163) (width 0.25) (layer F.Cu) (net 10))
 (segment (start 77.6527 93.7163) (end 77.2024 94.1666) (width 0.25) (layer F.Cu) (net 10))
 (segment (start 77.2024 94.1666) (end 77.2024 98.2637) (width 0.25) (layer F.Cu) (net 10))
 (segment (start 77.2024 98.2637) (end 78.1814 99.2427) (width 0.25) (layer F.Cu) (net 10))
 (segment (start 78.1814 99.2427) (end 78.74 99.2427) (width 0.25) (layer F.Cu) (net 10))
 (segment (start 78.74 100.33) (end 78.74 99.2427) (width 0.25) (layer F.Cu) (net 10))
 (segment (start 57.658 59.69) (end 58.7693 58.5787) (width 0.25) (layer B.Cu) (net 10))
 (segment (start 58.7693 58.5787) (end 77.8981 58.5787) (width 0.25) (layer B.Cu) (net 10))
 (segment (start 77.8981 58.5787) (end 77.8981 71.5869) (width 0.25) (layer B.Cu) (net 10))
 (segment (start 77.8981 71.5869) (end 76.32 73.165) (width 0.25) (layer B.Cu) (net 10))
 (segment (start 84.38 58.42) (end 78.0568 58.42) (width 0.25) (layer B.Cu) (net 10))
 (segment (start 78.0568 58.42) (end 77.8981 58.5787) (width 0.25) (layer B.Cu) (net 10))
 (segment (start 85.05 45.67) (end 83.8747 45.67) (width 0.25) (layer F.Cu) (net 10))
 (segment (start 84.38 58.42) (end 83.8747 57.9147) (width 0.25) (layer F.Cu) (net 10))
 (segment (start 83.8747 57.9147) (end 83.8747 45.67) (width 0.25) (layer F.Cu) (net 10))
 (segment (start 53.848 60.9964) (end 53.848 51.2744) (width 0.25) (layer F.Cu) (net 10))
 (segment (start 53.848 51.2744) (end 52.578 50.0044) (width 0.25) (layer F.Cu) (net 10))
 (segment (start 52.578 50.0044) (end 52.578 44.45) (width 0.25) (layer F.Cu) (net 10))
 (segment (start 55.118 44.45) (end 52.578 44.45) (width 0.25) (layer B.Cu) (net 10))
 (segment (start 58.928 45.7764) (end 58.928 44.1329) (width 0.25) (layer B.Cu) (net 10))
 (segment (start 58.928 44.1329) (end 58.1557 43.3606) (width 0.25) (layer B.Cu) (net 10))
 (segment (start 58.1557 43.3606) (end 56.2074 43.3606) (width 0.25) (layer B.Cu) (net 10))
 (segment (start 56.2074 43.3606) (end 55.118 44.45) (width 0.25) (layer B.Cu) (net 10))
 (segment (start 56.388 60.9964) (end 56.388 60.96) (width 0.25) (layer B.Cu) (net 10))
 (segment (start 56.388 60.96) (end 57.658 59.69) (width 0.25) (layer B.Cu) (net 10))
 (segment (start 91 45.67) (end 85.05 45.67) (width 0.25) (layer B.Cu) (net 10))
 (segment (start 56.388 60.9964) (end 53.848 60.9964) (width 0.25) (layer B.Cu) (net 10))
 (segment (start 78.74 97.79) (end 78.74 96.7027) (width 0.25) (layer F.Cu) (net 11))
 (segment (start 62.5961 45.3655) (end 62.5961 59.8683) (width 0.25) (layer F.Cu) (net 11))
 (segment (start 62.5961 59.8683) (end 61.468 60.9964) (width 0.25) (layer F.Cu) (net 11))
 (segment (start 60.198 44.45) (end 61.6806 44.45) (width 0.25) (layer F.Cu) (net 11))
 (segment (start 61.6806 44.45) (end 62.5961 45.3655) (width 0.25) (layer F.Cu) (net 11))
 (segment (start 78.74 96.7027) (end 78.1963 96.7027) (width 0.25) (layer F.Cu) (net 11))
 (segment (start 78.1963 96.7027) (end 77.6527 96.1591) (width 0.25) (layer F.Cu) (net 11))
 (segment (start 77.6527 96.1591) (end 77.6527 94.3532) (width 0.25) (layer F.Cu) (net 11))
 (segment (start 77.6527 94.3532) (end 78.3767 93.6292) (width 0.25) (layer F.Cu) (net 11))
 (segment (start 78.3767 93.6292) (end 78.3767 44.9221) (width 0.25) (layer F.Cu) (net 11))
 (segment (start 78.3767 44.9221) (end 77.3392 43.8846) (width 0.25) (layer F.Cu) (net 11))
 (segment (start 77.3392 43.8846) (end 64.077 43.8846) (width 0.25) (layer F.Cu) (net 11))
 (segment (start 64.077 43.8846) (end 62.5961 45.3655) (width 0.25) (layer F.Cu) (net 11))
 (segment (start 39.0353 73.1) (end 47.5628 64.5725) (width 0.25) (layer F.Cu) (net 12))
 (segment (start 47.5628 64.5725) (end 47.8189 64.5725) (width 0.25) (layer F.Cu) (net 12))
 (segment (start 47.8189 64.5725) (end 50.038 62.3534) (width 0.25) (layer F.Cu) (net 12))
 (segment (start 50.038 62.3534) (end 50.038 59.69) (width 0.25) (layer F.Cu) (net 12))
 (segment (start 37.46 73.1) (end 39.0353 73.1) (width 0.25) (layer F.Cu) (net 12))
 (segment (start 37.46 73.7626) (end 37.46 73.1) (width 0.25) (layer F.Cu) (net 12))
 (segment (start 37.46 73.7626) (end 37.46 74.4253) (width 0.25) (layer F.Cu) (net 12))
 (segment (start 37.46 94.57) (end 37.46 93.2447) (width 0.25) (layer F.Cu) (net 12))
 (segment (start 37.46 93.2447) (end 37.5259 93.1788) (width 0.25) (layer F.Cu) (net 12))
 (segment (start 37.5259 93.1788) (end 37.5259 74.4912) (width 0.25) (layer F.Cu) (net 12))
 (segment (start 37.5259 74.4912) (end 37.46 74.4253) (width 0.25) (layer F.Cu) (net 12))
 (segment (start 51.308 45.7764) (end 51.308 58.42) (width 0.25) (layer B.Cu) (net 12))
 (segment (start 51.308 58.42) (end 50.038 59.69) (width 0.25) (layer B.Cu) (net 12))
 (segment (start 58.93 94.57) (end 58.93 93.2447) (width 0.25) (layer B.Cu) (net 13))
 (segment (start 58.93 73.1) (end 58.93 74.4253) (width 0.25) (layer B.Cu) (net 13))
 (segment (start 58.93 74.4253) (end 58.9959 74.4912) (width 0.25) (layer B.Cu) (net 13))
 (segment (start 58.9959 74.4912) (end 58.9959 93.1788) (width 0.25) (layer B.Cu) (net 13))
 (segment (start 58.9959 93.1788) (end 58.93 93.2447) (width 0.25) (layer B.Cu) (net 13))
 (segment (start 47.498 63.8002) (end 56.7978 73.1) (width 0.25) (layer B.Cu) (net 13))
 (segment (start 56.7978 73.1) (end 58.93 73.1) (width 0.25) (layer B.Cu) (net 13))
 (segment (start 47.498 59.69) (end 47.498 63.8002) (width 0.25) (layer F.Cu) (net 13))
 (segment (start 48.768 45.7764) (end 48.768 58.42) (width 0.25) (layer B.Cu) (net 13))
 (segment (start 48.768 58.42) (end 47.498 59.69) (width 0.25) (layer B.Cu) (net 13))
 (via (at 47.498 63.8002) (size 0.8) (layers F.Cu B.Cu) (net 13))
 (segment (start 55.118 59.69) (end 57.7418 57.0662) (width 0.25) (layer B.Cu) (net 14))
 (segment (start 57.7418 57.0662) (end 89.5262 57.0662) (width 0.25) (layer B.Cu) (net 14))
 (segment (start 89.5262 57.0662) (end 90.88 58.42) (width 0.25) (layer B.Cu) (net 14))
 (segment (start 55.118 59.69) (end 55.118 47.0464) (width 0.25) (layer F.Cu) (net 14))
 (segment (start 55.118 47.0464) (end 56.388 45.7764) (width 0.25) (layer F.Cu) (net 14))
 (segment (start 32.258 59.69) (end 32.258 61.2905) (width 0.25) (layer B.Cu) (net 15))
 (segment (start 32.258 61.2905) (end 34.0416 63.0741) (width 0.25) (layer B.Cu) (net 15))
 (segment (start 34.0416 63.0741) (end 63.7291 63.0741) (width 0.25) (layer B.Cu) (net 15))
 (segment (start 63.7291 63.0741) (end 76.32 75.665) (width 0.25) (layer B.Cu) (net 15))
 (segment (start 32.258 59.69) (end 33.528 58.42) (width 0.25) (layer F.Cu) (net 15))
 (segment (start 33.528 58.42) (end 33.528 45.7764) (width 0.25) (layer F.Cu) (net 15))
 (segment (start 76.32 70.665) (end 74.9947 70.665) (width 0.25) (layer B.Cu) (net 16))
 (segment (start 74.9947 70.665) (end 66.9534 62.6237) (width 0.25) (layer B.Cu) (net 16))
 (segment (start 66.9534 62.6237) (end 36.1399 62.6237) (width 0.25) (layer B.Cu) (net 16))
 (segment (start 36.1399 62.6237) (end 34.798 61.2818) (width 0.25) (layer B.Cu) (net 16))
 (segment (start 34.798 61.2818) (end 34.798 59.69) (width 0.25) (layer B.Cu) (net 16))
 (segment (start 36.068 45.7764) (end 36.068 58.42) (width 0.25) (layer B.Cu) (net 16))
 (segment (start 36.068 58.42) (end 34.798 59.69) (width 0.25) (layer B.Cu) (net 16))
 (segment (start 60.198 59.69) (end 61.468 58.42) (width 0.25) (layer F.Cu) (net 17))
 (segment (start 61.468 58.42) (end 61.468 45.7764) (width 0.25) (layer F.Cu) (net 17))
 (segment (start 44.958 59.69) (end 44.958 47.0464) (width 0.25) (layer B.Cu) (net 18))
 (segment (start 44.958 47.0464) (end 46.228 45.7764) (width 0.25) (layer B.Cu) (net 18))
 (segment (start 43.688 45.7764) (end 43.688 58.42) (width 0.25) (layer B.Cu) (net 19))
 (segment (start 43.688 58.42) (end 42.418 59.69) (width 0.25) (layer B.Cu) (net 19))
 (segment (start 41.148 45.7764) (end 41.148 58.42) (width 0.25) (layer B.Cu) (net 20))
 (segment (start 41.148 58.42) (end 39.878 59.69) (width 0.25) (layer B.Cu) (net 20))
 (segment (start 38.608 45.7764) (end 38.608 58.42) (width 0.25) (layer B.Cu) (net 21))
 (segment (start 38.608 58.42) (end 37.338 59.69) (width 0.25) (layer B.Cu) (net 21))
 (segment (start 32.258 44.45) (end 32.258 51.8919) (width 0.25) (layer B.Cu) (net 22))
 (segment (start 32.258 51.8919) (end 33.528 53.1619) (width 0.25) (layer B.Cu) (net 22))
 (segment (start 33.528 53.1619) (end 33.528 60.9964) (width 0.25) (layer B.Cu) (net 22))
 (segment (start 34.798 44.45) (end 34.798 51.8919) (width 0.25) (layer F.Cu) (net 23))
 (segment (start 34.798 51.8919) (end 36.068 53.1619) (width 0.25) (layer F.Cu) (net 23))
 (segment (start 36.068 53.1619) (end 36.068 60.9964) (width 0.25) (layer F.Cu) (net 23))
 (segment (start 37.338 44.45) (end 37.338 51.8919) (width 0.25) (layer F.Cu) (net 24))
 (segment (start 37.338 51.8919) (end 38.608 53.1619) (width 0.25) (layer F.Cu) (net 24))
 (segment (start 38.608 53.1619) (end 38.608 60.9964) (width 0.25) (layer F.Cu) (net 24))
 (segment (start 39.878 44.45) (end 39.878 51.8919) (width 0.25) (layer F.Cu) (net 25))
 (segment (start 39.878 51.8919) (end 41.148 53.1619) (width 0.25) (layer F.Cu) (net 25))
 (segment (start 41.148 53.1619) (end 41.148 60.9964) (width 0.25) (layer F.Cu) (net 25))
 (segment (start 47.498 44.45) (end 47.498 51.8919) (width 0.25) (layer F.Cu) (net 26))
 (segment (start 47.498 51.8919) (end 48.768 53.1619) (width 0.25) (layer F.Cu) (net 26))
 (segment (start 48.768 53.1619) (end 48.768 60.9964) (width 0.25) (layer F.Cu) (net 26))
 (segment (start 50.038 44.45) (end 50.038 51.8919) (width 0.25) (layer F.Cu) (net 27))
 (segment (start 50.038 51.8919) (end 51.308 53.1619) (width 0.25) (layer F.Cu) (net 27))
 (segment (start 51.308 53.1619) (end 51.308 60.9964) (width 0.25) (layer F.Cu) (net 27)))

